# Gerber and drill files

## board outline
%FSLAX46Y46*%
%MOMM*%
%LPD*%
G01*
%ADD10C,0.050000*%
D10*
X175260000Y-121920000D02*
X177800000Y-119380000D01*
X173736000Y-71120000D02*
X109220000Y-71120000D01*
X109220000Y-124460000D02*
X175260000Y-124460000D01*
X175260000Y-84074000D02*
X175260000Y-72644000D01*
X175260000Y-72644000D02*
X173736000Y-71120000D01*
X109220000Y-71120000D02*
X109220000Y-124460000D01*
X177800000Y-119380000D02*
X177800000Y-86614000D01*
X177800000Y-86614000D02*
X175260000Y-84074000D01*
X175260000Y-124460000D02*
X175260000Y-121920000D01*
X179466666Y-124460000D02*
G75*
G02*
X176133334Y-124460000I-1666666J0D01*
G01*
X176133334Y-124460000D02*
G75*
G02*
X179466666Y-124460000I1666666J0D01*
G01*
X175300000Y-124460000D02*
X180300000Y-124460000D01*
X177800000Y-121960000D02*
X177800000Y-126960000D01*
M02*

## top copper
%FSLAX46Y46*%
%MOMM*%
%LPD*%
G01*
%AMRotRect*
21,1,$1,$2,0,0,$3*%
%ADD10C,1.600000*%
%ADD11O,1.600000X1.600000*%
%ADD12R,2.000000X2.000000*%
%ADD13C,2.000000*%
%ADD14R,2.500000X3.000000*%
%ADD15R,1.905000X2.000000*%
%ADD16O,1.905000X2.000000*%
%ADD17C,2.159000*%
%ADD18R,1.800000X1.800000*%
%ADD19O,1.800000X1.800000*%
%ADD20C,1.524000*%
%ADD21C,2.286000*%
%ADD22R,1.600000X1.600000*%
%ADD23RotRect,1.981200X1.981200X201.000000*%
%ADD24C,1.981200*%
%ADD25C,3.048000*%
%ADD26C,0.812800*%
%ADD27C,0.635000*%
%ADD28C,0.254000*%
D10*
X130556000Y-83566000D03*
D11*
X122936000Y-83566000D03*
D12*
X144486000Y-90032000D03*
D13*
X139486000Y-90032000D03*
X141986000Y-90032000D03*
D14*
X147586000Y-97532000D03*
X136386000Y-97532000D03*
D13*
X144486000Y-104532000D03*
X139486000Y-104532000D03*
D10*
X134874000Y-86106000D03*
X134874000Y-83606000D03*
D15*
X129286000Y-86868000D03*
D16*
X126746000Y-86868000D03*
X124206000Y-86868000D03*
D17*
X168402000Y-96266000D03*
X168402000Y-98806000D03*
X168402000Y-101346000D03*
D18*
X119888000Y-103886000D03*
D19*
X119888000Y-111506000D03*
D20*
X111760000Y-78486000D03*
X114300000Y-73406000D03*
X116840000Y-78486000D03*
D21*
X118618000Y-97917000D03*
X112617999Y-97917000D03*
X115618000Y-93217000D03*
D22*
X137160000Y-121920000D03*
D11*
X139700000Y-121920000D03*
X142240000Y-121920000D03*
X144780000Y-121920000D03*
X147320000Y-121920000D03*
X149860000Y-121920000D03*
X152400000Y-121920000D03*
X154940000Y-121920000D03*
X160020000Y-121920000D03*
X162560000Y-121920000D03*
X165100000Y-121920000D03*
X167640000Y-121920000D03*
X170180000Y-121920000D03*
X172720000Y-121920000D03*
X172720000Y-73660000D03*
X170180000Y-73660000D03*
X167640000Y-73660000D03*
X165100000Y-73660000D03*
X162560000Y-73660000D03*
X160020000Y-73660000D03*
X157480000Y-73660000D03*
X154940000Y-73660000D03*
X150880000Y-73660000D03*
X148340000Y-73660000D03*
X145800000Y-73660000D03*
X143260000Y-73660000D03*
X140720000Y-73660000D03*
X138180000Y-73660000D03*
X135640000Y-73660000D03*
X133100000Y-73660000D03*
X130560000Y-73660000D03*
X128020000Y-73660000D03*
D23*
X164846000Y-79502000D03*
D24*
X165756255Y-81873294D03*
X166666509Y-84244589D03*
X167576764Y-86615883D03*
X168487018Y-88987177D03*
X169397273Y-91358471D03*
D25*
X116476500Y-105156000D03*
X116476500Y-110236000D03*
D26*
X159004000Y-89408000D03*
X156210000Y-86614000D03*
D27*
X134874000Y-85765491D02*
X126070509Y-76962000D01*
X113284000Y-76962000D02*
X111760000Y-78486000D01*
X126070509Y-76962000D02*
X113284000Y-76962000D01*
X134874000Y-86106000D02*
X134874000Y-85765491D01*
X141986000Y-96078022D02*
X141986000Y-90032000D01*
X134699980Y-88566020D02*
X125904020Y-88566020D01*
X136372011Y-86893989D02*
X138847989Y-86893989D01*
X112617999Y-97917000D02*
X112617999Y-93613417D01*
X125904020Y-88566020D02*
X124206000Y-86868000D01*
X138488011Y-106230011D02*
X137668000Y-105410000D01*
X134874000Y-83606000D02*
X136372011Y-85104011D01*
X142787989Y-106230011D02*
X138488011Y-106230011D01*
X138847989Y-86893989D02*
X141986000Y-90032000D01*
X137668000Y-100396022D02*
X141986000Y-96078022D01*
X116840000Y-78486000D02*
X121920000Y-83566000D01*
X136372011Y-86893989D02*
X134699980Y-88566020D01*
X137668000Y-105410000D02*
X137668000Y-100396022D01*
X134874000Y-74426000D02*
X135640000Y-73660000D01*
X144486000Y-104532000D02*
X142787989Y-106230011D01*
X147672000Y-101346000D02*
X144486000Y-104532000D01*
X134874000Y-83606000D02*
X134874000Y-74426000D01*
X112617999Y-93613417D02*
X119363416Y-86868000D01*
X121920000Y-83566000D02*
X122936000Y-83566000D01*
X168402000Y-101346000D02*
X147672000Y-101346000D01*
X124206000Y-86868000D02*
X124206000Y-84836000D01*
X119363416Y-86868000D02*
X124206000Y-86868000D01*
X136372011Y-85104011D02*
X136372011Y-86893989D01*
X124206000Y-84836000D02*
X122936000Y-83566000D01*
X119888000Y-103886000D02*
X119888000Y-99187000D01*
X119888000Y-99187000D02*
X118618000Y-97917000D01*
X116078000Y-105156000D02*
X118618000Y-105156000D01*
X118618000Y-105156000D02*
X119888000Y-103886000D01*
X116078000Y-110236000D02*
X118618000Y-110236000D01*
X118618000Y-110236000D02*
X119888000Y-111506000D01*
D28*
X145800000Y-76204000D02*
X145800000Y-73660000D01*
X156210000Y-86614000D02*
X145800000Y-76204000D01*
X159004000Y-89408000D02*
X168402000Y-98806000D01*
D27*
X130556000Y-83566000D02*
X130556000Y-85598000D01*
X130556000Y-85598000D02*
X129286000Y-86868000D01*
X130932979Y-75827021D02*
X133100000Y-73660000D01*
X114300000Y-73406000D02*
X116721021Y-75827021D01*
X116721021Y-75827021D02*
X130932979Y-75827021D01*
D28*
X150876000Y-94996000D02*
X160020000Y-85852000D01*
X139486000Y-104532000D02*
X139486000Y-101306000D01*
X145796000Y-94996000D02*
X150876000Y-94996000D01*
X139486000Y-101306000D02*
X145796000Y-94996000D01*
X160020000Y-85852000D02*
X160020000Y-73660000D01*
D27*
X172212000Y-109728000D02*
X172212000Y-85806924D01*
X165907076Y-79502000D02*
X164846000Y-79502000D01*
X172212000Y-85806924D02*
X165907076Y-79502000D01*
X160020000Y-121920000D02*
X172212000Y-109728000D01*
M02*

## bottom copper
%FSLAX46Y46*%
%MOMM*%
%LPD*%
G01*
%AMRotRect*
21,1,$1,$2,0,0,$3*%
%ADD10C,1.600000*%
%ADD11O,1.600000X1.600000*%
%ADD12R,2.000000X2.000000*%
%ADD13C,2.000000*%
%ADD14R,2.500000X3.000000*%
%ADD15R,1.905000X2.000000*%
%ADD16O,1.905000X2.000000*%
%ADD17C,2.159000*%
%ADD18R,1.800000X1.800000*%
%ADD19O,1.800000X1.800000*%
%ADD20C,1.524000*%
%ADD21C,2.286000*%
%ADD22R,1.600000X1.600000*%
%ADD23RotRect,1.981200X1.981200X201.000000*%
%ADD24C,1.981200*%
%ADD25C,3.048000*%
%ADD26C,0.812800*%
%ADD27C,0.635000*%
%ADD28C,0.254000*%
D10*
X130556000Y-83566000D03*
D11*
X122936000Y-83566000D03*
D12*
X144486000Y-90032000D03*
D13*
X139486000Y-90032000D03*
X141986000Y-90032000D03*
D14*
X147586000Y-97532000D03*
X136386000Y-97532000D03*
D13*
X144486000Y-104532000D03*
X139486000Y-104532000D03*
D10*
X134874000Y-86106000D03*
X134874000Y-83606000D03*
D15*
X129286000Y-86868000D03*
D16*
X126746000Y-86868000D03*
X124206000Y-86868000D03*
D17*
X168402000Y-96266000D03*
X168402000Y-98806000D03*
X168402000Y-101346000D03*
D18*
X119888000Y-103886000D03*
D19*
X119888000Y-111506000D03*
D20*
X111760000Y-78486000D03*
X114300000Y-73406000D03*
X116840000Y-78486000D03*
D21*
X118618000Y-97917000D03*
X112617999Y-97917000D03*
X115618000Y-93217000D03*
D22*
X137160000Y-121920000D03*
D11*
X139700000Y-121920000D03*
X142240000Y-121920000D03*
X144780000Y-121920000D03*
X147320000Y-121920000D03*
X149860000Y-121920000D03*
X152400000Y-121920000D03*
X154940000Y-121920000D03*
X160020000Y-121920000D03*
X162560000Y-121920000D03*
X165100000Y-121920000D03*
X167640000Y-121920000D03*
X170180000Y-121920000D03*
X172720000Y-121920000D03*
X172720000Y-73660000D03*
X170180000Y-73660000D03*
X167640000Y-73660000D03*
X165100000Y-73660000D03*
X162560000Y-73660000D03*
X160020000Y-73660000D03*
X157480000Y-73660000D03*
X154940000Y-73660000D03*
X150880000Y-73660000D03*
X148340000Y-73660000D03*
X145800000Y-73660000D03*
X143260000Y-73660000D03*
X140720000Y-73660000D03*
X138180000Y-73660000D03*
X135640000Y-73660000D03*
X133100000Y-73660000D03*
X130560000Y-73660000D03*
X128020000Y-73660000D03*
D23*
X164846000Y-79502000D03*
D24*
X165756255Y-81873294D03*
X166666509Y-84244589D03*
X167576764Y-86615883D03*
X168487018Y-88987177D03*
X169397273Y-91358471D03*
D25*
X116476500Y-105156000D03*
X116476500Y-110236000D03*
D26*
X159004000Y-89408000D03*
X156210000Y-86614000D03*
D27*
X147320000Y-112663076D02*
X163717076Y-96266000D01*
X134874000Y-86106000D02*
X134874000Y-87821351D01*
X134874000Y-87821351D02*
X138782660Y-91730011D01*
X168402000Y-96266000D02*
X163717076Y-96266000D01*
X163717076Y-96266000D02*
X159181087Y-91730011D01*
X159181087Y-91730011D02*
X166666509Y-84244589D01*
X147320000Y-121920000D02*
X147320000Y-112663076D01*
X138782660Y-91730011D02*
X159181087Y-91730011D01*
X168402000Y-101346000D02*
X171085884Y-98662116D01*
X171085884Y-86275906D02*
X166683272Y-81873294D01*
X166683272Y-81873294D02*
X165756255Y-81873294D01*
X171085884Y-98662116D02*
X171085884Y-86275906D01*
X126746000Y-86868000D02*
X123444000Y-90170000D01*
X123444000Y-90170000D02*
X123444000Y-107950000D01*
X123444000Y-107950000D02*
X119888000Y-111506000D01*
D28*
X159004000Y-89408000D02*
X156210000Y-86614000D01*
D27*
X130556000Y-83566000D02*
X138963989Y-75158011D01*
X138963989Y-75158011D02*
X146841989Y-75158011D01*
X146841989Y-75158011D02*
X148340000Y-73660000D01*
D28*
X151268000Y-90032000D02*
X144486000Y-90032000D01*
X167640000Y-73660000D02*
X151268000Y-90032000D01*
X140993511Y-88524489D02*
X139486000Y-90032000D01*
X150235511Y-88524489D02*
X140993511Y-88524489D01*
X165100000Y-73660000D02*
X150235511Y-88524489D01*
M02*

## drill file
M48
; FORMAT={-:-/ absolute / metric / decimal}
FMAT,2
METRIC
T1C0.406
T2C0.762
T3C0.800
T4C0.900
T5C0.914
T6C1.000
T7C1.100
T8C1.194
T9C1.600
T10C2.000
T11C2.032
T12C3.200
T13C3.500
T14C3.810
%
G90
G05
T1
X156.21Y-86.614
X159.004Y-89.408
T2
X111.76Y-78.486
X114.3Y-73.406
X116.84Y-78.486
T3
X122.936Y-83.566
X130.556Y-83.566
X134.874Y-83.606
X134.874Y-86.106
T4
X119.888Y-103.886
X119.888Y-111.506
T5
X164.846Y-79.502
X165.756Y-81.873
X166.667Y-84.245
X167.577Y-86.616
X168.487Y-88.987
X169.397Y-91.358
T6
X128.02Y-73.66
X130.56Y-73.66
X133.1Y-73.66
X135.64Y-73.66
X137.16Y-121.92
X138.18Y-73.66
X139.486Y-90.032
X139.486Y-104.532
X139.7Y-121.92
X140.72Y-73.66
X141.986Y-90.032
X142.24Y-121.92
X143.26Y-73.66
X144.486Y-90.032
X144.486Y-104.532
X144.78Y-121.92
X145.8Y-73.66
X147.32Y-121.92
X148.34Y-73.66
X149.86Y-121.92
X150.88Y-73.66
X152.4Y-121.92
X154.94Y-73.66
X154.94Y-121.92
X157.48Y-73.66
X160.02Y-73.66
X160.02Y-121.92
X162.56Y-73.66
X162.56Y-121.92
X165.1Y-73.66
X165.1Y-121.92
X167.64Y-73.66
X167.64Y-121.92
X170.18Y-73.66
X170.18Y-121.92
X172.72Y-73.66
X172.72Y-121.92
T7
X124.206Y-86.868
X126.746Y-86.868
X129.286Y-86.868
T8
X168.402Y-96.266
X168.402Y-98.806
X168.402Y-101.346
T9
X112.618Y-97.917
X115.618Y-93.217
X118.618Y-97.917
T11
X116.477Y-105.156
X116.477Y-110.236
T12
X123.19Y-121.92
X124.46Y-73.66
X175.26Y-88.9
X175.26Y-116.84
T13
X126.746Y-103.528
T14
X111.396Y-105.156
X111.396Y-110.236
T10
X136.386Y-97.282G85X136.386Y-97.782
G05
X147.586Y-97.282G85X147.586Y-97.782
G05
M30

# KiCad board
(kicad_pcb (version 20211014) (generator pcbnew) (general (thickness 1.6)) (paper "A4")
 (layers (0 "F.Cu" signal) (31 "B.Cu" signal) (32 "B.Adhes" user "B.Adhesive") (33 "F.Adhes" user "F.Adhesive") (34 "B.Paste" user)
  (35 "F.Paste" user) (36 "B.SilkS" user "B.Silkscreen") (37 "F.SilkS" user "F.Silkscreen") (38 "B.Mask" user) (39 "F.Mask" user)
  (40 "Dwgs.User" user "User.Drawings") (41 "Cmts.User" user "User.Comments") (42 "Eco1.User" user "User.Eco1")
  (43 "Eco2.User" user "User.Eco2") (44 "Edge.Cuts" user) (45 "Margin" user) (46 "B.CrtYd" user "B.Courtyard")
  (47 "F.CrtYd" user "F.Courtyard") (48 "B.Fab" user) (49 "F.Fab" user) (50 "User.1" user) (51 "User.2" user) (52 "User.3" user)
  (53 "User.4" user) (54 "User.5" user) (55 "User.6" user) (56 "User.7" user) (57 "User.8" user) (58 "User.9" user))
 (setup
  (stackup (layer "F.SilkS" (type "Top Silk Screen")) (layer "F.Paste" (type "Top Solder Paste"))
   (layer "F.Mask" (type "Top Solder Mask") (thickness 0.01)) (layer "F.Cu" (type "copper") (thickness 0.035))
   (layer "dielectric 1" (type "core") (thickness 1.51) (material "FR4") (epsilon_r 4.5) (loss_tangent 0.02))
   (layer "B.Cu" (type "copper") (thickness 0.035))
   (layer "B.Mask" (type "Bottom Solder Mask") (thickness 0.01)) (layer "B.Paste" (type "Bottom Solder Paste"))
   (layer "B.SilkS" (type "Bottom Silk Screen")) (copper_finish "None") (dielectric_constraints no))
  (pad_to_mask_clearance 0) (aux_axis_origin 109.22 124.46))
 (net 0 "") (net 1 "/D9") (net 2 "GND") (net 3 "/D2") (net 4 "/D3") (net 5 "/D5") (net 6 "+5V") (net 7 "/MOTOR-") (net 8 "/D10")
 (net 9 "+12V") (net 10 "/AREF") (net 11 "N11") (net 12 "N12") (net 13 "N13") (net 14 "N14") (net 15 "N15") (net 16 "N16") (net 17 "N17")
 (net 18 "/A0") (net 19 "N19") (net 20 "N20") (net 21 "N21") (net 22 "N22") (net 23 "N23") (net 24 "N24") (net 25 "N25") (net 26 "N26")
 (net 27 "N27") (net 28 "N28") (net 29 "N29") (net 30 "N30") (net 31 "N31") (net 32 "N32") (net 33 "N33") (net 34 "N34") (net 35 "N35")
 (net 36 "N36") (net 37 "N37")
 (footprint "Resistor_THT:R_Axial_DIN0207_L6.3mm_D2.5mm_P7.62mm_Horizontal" (layer "F.Cu") (at 130.556 83.566 180)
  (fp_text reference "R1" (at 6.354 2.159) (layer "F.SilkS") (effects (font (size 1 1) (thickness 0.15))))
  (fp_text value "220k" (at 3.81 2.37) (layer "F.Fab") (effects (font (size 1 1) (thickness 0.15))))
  (pad "1" thru_hole circle (at 0 0 180) (size 1.6 1.6) (drill 0.8) (layers *.Cu *.Mask) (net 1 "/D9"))
  (pad "2" thru_hole oval (at 7.62 0 180) (size 1.6 1.6) (drill 0.8) (layers *.Cu *.Mask) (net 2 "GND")))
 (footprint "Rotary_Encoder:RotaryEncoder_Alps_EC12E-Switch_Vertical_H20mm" (layer "F.Cu") (at 144.486 90.032 -90)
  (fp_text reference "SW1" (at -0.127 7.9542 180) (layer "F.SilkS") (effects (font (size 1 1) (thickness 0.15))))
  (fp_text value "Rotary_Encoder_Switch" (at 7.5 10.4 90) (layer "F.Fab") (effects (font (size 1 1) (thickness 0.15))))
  (pad "A" thru_hole rect (at 0 0 270) (size 2 2) (drill 1) (layers *.Cu *.Mask) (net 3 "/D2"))
  (pad "B" thru_hole circle (at 0 5 270) (size 2 2) (drill 1) (layers *.Cu *.Mask) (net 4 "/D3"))
  (pad "C" thru_hole circle (at 0 2.5 270) (size 2 2) (drill 1) (layers *.Cu *.Mask) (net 2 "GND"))
  (pad "MP" thru_hole rect (at 7.5 -3.1 270) (size 3 2.5) (drill oval 2.5 2) (layers *.Cu *.Mask))
  (pad "MP" thru_hole rect (at 7.5 8.1 270) (size 3 2.5) (drill oval 2.5 2) (layers *.Cu *.Mask))
  (pad "S1" thru_hole circle (at 14.5 0 270) (size 2 2) (drill 1) (layers *.Cu *.Mask) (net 2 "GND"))
  (pad "S2" thru_hole circle (at 14.5 5 270) (size 2 2) (drill 1) (layers *.Cu *.Mask) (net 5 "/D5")))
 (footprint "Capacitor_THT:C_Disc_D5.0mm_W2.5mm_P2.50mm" (layer "F.Cu") (at 134.874 86.106 90)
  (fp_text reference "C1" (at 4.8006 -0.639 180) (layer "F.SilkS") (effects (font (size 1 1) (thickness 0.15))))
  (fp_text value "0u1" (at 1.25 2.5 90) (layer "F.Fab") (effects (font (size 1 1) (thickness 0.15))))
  (pad "1" thru_hole circle (at 0 0 90) (size 1.6 1.6) (drill 0.8) (layers *.Cu *.Mask) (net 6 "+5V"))
  (pad "2" thru_hole circle (at 2.5 0 90) (size 1.6 1.6) (drill 0.8) (layers *.Cu *.Mask) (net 2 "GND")))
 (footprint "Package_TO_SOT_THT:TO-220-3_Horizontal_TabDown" (layer "F.Cu") (at 129.286 86.868 180)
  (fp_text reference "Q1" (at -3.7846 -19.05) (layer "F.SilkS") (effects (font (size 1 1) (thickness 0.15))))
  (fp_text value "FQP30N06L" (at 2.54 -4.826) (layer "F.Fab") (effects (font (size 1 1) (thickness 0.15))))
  (pad "" np_thru_hole oval (at 2.54 -16.66 180) (size 3.5 3.5) (drill 3.5) (layers *.Cu *.Mask))
  (pad "1" thru_hole rect (at 0 0 180) (size 1.905 2) (drill 1.1) (layers *.Cu *.Mask) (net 1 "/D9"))
  (pad "2" thru_hole oval (at 2.54 0 180) (size 1.905 2) (drill 1.1) (layers *.Cu *.Mask) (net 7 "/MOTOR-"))
  (pad "3" thru_hole oval (at 5.08 0 180) (size 1.905 2) (drill 1.1) (layers *.Cu *.Mask) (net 2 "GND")))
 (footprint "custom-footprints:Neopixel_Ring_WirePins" (layer "F.Cu") (at 168.402 96.266)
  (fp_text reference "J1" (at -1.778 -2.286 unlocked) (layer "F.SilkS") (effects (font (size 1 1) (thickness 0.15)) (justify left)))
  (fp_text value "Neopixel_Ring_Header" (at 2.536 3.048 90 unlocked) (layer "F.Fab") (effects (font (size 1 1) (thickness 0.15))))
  (pad "1" thru_hole circle (at 0 0) (size 2.159 2.159) (drill 1.1938) (layers *.Cu *.Mask) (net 6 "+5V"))
  (pad "2" thru_hole circle (at 0 2.54) (size 2.159 2.159) (drill 1.1938) (layers *.Cu *.Mask) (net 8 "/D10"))
  (pad "3" thru_hole circle (at 0 5.08) (size 2.159 2.159) (drill 1.1938) (layers *.Cu *.Mask) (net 2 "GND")))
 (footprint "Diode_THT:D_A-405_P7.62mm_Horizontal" (layer "F.Cu") (at 119.888 103.886 -90)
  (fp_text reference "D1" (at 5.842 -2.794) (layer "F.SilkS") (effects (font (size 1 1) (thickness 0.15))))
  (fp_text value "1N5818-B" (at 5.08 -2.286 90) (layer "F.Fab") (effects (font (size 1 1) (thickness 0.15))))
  (pad "1" thru_hole rect (at 0 0 270) (size 1.8 1.8) (drill 0.9) (layers *.Cu *.Mask) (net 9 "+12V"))
  (pad "2" thru_hole oval (at 7.62 0 270) (size 1.8 1.8) (drill 0.9) (layers *.Cu *.Mask) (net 7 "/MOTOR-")))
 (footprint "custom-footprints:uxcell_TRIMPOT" (layer "F.Cu") (at 111.76 78.486)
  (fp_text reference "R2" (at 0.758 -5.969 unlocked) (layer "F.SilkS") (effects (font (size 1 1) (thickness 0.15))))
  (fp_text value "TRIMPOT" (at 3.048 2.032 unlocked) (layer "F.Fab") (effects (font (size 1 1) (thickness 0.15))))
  (pad "1" thru_hole circle (at 0 0) (size 1.524 1.524) (drill 0.762) (layers *.Cu *.Mask) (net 6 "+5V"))
  (pad "2" thru_hole circle (at 2.54 -5.08) (size 1.524 1.524) (drill 0.762) (layers *.Cu *.Mask) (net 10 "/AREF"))
  (pad "3" thru_hole circle (at 5.08 0) (size 1.524 1.524) (drill 0.762) (layers *.Cu *.Mask) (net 2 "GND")))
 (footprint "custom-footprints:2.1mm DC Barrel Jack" (layer "B.Cu") (at 118.618 97.917 -90)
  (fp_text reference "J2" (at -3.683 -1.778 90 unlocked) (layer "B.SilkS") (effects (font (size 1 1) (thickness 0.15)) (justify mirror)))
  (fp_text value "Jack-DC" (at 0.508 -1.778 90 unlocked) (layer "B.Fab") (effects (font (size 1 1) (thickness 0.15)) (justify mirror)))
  (pad "1" thru_hole circle (at 0 0 270) (size 2.286 2.286) (drill 1.6002) (layers *.Cu *.Mask) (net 9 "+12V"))
  (pad "2" thru_hole circle (at 0 6.000001 270) (size 2.286 2.286) (drill 1.6002) (layers *.Cu *.Mask) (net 2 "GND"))
  (pad "3" thru_hole circle (at -4.7 3 270) (size 2.286 2.286) (drill 1.6002) (layers *.Cu *.Mask)))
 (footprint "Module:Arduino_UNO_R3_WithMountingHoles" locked (layer "B.Cu") (at 137.16 121.92)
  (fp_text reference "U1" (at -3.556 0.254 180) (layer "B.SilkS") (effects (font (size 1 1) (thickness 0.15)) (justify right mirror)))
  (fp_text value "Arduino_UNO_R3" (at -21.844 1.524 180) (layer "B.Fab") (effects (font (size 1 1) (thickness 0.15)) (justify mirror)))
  (pad "" np_thru_hole circle locked (at -12.7 -48.26 270) (size 3.2 3.2) (drill 3.2) (layers *.Cu *.Mask))
  (pad "" np_thru_hole circle locked (at 38.1 -5.08 270) (size 3.2 3.2) (drill 3.2) (layers *.Cu *.Mask))
  (pad "" np_thru_hole circle locked (at -13.97 0 270) (size 3.2 3.2) (drill 3.2) (layers *.Cu *.Mask))
  (pad "" np_thru_hole circle locked (at 38.1 -33.02 270) (size 3.2 3.2) (drill 3.2) (layers *.Cu *.Mask))
  (pad "1" thru_hole rect locked (at 0 0 270) (size 1.6 1.6) (drill 1) (layers *.Cu *.Mask) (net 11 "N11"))
  (pad "2" thru_hole oval locked (at 2.54 0 270) (size 1.6 1.6) (drill 1) (layers *.Cu *.Mask) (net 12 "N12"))
  (pad "3" thru_hole oval locked (at 5.08 0 270) (size 1.6 1.6) (drill 1) (layers *.Cu *.Mask) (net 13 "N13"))
  (pad "4" thru_hole oval locked (at 7.62 0 270) (size 1.6 1.6) (drill 1) (layers *.Cu *.Mask) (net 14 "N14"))
  (pad "5" thru_hole oval locked (at 10.16 0 270) (size 1.6 1.6) (drill 1) (layers *.Cu *.Mask) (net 6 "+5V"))
  (pad "6" thru_hole oval locked (at 12.7 0 270) (size 1.6 1.6) (drill 1) (layers *.Cu *.Mask) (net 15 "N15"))
  (pad "7" thru_hole oval locked (at 15.24 0 270) (size 1.6 1.6) (drill 1) (layers *.Cu *.Mask) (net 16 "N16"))
  (pad "8" thru_hole oval locked (at 17.78 0 270) (size 1.6 1.6) (drill 1) (layers *.Cu *.Mask) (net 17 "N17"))
  (pad "9" thru_hole oval locked (at 22.86 0 270) (size 1.6 1.6) (drill 1) (layers *.Cu *.Mask) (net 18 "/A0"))
  (pad "10" thru_hole oval locked (at 25.4 0 270) (size 1.6 1.6) (drill 1) (layers *.Cu *.Mask) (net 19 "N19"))
  (pad "11" thru_hole oval locked (at 27.94 0 270) (size 1.6 1.6) (drill 1) (layers *.Cu *.Mask) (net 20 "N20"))
  (pad "12" thru_hole oval locked (at 30.48 0 270) (size 1.6 1.6) (drill 1) (layers *.Cu *.Mask) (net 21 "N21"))
  (pad "13" thru_hole oval locked (at 33.02 0 270) (size 1.6 1.6) (drill 1) (layers *.Cu *.Mask) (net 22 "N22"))
  (pad "14" thru_hole oval locked (at 35.56 0 270) (size 1.6 1.6) (drill 1) (layers *.Cu *.Mask) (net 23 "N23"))
  (pad "15" thru_hole oval locked (at 35.56 -48.26 270) (size 1.6 1.6) (drill 1) (layers *.Cu *.Mask) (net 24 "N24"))
  (pad "16" thru_hole oval locked (at 33.02 -48.26 270) (size 1.6 1.6) (drill 1) (layers *.Cu *.Mask) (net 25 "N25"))
  (pad "17" thru_hole oval locked (at 30.48 -48.26 270) (size 1.6 1.6) (drill 1) (layers *.Cu *.Mask) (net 3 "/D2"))
  (pad "18" thru_hole oval locked (at 27.94 -48.26 270) (size 1.6 1.6) (drill 1) (layers *.Cu *.Mask) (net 4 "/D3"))
  (pad "19" thru_hole oval locked (at 25.4 -48.26 270) (size 1.6 1.6) (drill 1) (layers *.Cu *.Mask) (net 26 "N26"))
  (pad "20" thru_hole oval locked (at 22.86 -48.26 270) (size 1.6 1.6) (drill 1) (layers *.Cu *.Mask) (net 5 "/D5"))
  (pad "21" thru_hole oval locked (at 20.32 -48.26 270) (size 1.6 1.6) (drill 1) (layers *.Cu *.Mask) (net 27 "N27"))
  (pad "22" thru_hole oval locked (at 17.78 -48.26 270) (size 1.6 1.6) (drill 1) (layers *.Cu *.Mask) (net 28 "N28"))
  (pad "23" thru_hole oval locked (at 13.72 -48.26 270) (size 1.6 1.6) (drill 1) (layers *.Cu *.Mask) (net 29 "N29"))
  (pad "24" thru_hole oval locked (at 11.18 -48.26 270) (size 1.6 1.6) (drill 1) (layers *.Cu *.Mask) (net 1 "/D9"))
  (pad "25" thru_hole oval locked (at 8.64 -48.26 270) (size 1.6 1.6) (drill 1) (layers *.Cu *.Mask) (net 8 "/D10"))
  (pad "26" thru_hole oval locked (at 6.1 -48.26 270) (size 1.6 1.6) (drill 1) (layers *.Cu *.Mask) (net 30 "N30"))
  (pad "27" thru_hole oval locked (at 3.56 -48.26 270) (size 1.6 1.6) (drill 1) (layers *.Cu *.Mask) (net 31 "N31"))
  (pad "28" thru_hole oval locked (at 1.02 -48.26 270) (size 1.6 1.6) (drill 1) (layers *.Cu *.Mask) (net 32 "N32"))
  (pad "29" thru_hole oval locked (at -1.52 -48.26 270) (size 1.6 1.6) (drill 1) (layers *.Cu *.Mask) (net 2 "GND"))
  (pad "30" thru_hole oval locked (at -4.06 -48.26 270) (size 1.6 1.6) (drill 1) (layers *.Cu *.Mask) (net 10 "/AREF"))
  (pad "31" thru_hole oval locked (at -6.6 -48.26 270) (size 1.6 1.6) (drill 1) (layers *.Cu *.Mask) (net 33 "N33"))
  (pad "32" thru_hole oval locked (at -9.14 -48.26 270) (size 1.6 1.6) (drill 1) (layers *.Cu *.Mask) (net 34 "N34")))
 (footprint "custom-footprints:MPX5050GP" (layer "B.Cu") (at 164.846 79.502 -159)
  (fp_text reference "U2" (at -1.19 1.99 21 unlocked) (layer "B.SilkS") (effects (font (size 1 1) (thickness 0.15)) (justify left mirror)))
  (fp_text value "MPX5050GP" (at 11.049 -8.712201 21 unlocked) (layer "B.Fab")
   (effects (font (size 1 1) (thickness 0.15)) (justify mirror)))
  (pad "1" thru_hole rect (at 0 0 201) (size 1.9812 1.9812) (drill 0.9144) (layers *.Cu *.Mask) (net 18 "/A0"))
  (pad "2" thru_hole circle (at 0 -2.54 201) (size 1.9812 1.9812) (drill 0.9144) (layers *.Cu *.Mask) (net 2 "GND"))
  (pad "3" thru_hole circle (at 0 -5.08 201) (size 1.9812 1.9812) (drill 0.9144) (layers *.Cu *.Mask) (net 6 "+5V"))
  (pad "4" thru_hole circle (at 0 -7.62 201) (size 1.9812 1.9812) (drill 0.9144) (layers *.Cu *.Mask) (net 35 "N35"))
  (pad "5" thru_hole circle (at 0 -10.16 201) (size 1.9812 1.9812) (drill 0.9144) (layers *.Cu *.Mask) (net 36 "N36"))
  (pad "6" thru_hole circle (at 0 -12.7 201) (size 1.9812 1.9812) (drill 0.9144) (layers *.Cu *.Mask) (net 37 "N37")))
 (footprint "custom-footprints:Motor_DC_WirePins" (layer "B.Cu") (at 116.4765 105.156 180)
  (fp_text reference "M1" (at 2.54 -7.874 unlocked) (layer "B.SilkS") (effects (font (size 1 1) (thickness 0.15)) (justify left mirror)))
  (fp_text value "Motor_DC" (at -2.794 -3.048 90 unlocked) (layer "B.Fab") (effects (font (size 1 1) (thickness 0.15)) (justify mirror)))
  (pad "" np_thru_hole circle (at 5.08 0 180) (size 3.302 3.302) (drill 3.81) (layers *.Mask))
  (pad "" np_thru_hole circle (at 5.08 -5.08 180) (size 3.302 3.302) (drill 3.81) (layers *.Mask))
  (pad "1" thru_hole circle (at 0 0 180) (size 3.048 3.048) (drill 2.032) (layers *.Cu *.Mask) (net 9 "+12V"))
  (pad "2" thru_hole circle (at 0 -5.08 180) (size 3.048 3.048) (drill 2.032) (layers *.Cu *.Mask) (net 7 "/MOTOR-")))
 (gr_line (start 175.26 121.92) (end 177.8 119.38) (layer "Edge.Cuts") (width 0.05))
 (gr_line (start 173.736 71.12) (end 109.22 71.12) (layer "Edge.Cuts") (width 0.05))
 (gr_line (start 109.22 124.46) (end 175.26 124.46) (layer "Edge.Cuts") (width 0.05))
 (gr_line (start 175.26 84.074) (end 175.26 72.644) (layer "Edge.Cuts") (width 0.05))
 (gr_line (start 175.26 72.644) (end 173.736 71.12) (layer "Edge.Cuts") (width 0.05))
 (gr_line (start 109.22 71.12) (end 109.22 124.46) (layer "Edge.Cuts") (width 0.05))
 (gr_line (start 177.8 119.38) (end 177.8 86.614) (layer "Edge.Cuts") (width 0.05))
 (gr_line (start 177.8 86.614) (end 175.26 84.074) (layer "Edge.Cuts") (width 0.05))
 (gr_line (start 175.26 124.46) (end 175.26 121.92) (layer "Edge.Cuts") (width 0.05))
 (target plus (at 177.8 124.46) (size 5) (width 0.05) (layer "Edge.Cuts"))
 (segment (start 134.874 85.765491) (end 126.070509 76.962) (width 0.635) (layer "F.Cu") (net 6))
 (segment (start 113.284 76.962) (end 111.76 78.486) (width 0.635) (layer "F.Cu") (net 6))
 (segment (start 126.070509 76.962) (end 113.284 76.962) (width 0.635) (layer "F.Cu") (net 6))
 (segment (start 134.874 86.106) (end 134.874 85.765491) (width 0.635) (layer "F.Cu") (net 6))
 (segment (start 147.32 112.663076) (end 163.717076 96.266) (width 0.635) (layer "B.Cu") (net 6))
 (segment (start 134.874 86.106) (end 134.874 87.821351) (width 0.635) (layer "B.Cu") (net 6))
 (segment (start 134.874 87.821351) (end 138.78266 91.730011) (width 0.635) (layer "B.Cu") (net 6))
 (segment (start 168.402 96.266) (end 163.717076 96.266) (width 0.635) (layer "B.Cu") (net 6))
 (segment (start 163.717076 96.266) (end 159.181087 91.730011) (width 0.635) (layer "B.Cu") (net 6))
 (segment (start 159.181087 91.730011) (end 166.666509 84.244589) (width 0.635) (layer "B.Cu") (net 6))
 (segment (start 147.32 121.92) (end 147.32 112.663076) (width 0.635) (layer "B.Cu") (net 6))
 (segment (start 138.78266 91.730011) (end 159.181087 91.730011) (width 0.635) (layer "B.Cu") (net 6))
 (segment (start 141.986 96.078022) (end 141.986 90.032) (width 0.635) (layer "F.Cu") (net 2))
 (segment (start 134.69998 88.56602) (end 125.90402 88.56602) (width 0.635) (layer "F.Cu") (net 2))
 (segment (start 136.372011 86.893989) (end 138.847989 86.893989) (width 0.635) (layer "F.Cu") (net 2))
 (segment (start 112.617999 97.917) (end 112.617999 93.613417) (width 0.635) (layer "F.Cu") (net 2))
 (segment (start 125.90402 88.56602) (end 124.206 86.868) (width 0.635) (layer "F.Cu") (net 2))
 (segment (start 138.488011 106.230011) (end 137.668 105.41) (width 0.635) (layer "F.Cu") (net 2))
 (segment (start 134.874 83.606) (end 136.372011 85.104011) (width 0.635) (layer "F.Cu") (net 2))
 (segment (start 142.787989 106.230011) (end 138.488011 106.230011) (width 0.635) (layer "F.Cu") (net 2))
 (segment (start 138.847989 86.893989) (end 141.986 90.032) (width 0.635) (layer "F.Cu") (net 2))
 (segment (start 137.668 100.396022) (end 141.986 96.078022) (width 0.635) (layer "F.Cu") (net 2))
 (segment (start 116.84 78.486) (end 121.92 83.566) (width 0.635) (layer "F.Cu") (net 2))
 (segment (start 136.372011 86.893989) (end 134.69998 88.56602) (width 0.635) (layer "F.Cu") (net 2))
 (segment (start 137.668 105.41) (end 137.668 100.396022) (width 0.635) (layer "F.Cu") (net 2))
 (segment (start 134.874 74.426) (end 135.64 73.66) (width 0.635) (layer "F.Cu") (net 2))
 (segment (start 144.486 104.532) (end 142.787989 106.230011) (width 0.635) (layer "F.Cu") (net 2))
 (segment (start 147.672 101.346) (end 144.486 104.532) (width 0.635) (layer "F.Cu") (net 2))
 (segment (start 134.874 83.606) (end 134.874 74.426) (width 0.635) (layer "F.Cu") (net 2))
 (segment (start 112.617999 93.613417) (end 119.363416 86.868) (width 0.635) (layer "F.Cu") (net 2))
 (segment (start 121.92 83.566) (end 122.936 83.566) (width 0.635) (layer "F.Cu") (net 2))
 (segment (start 168.402 101.346) (end 147.672 101.346) (width 0.635) (layer "F.Cu") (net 2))
 (segment (start 124.206 86.868) (end 124.206 84.836) (width 0.635) (layer "F.Cu") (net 2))
 (segment (start 119.363416 86.868) (end 124.206 86.868) (width 0.635) (layer "F.Cu") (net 2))
 (segment (start 136.372011 85.104011) (end 136.372011 86.893989) (width 0.635) (layer "F.Cu") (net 2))
 (segment (start 124.206 84.836) (end 122.936 83.566) (width 0.635) (layer "F.Cu") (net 2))
 (segment (start 168.402 101.346) (end 171.085884 98.662116) (width 0.635) (layer "B.Cu") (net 2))
 (segment (start 171.085884 86.275906) (end 166.683272 81.873294) (width 0.635) (layer "B.Cu") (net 2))
 (segment (start 166.683272 81.873294) (end 165.756255 81.873294) (width 0.635) (layer "B.Cu") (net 2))
 (segment (start 171.085884 98.662116) (end 171.085884 86.275906) (width 0.635) (layer "B.Cu") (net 2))
 (segment (start 119.888 103.886) (end 119.888 99.187) (width 0.635) (layer "F.Cu") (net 9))
 (segment (start 119.888 99.187) (end 118.618 97.917) (width 0.635) (layer "F.Cu") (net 9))
 (segment (start 116.078 105.156) (end 118.618 105.156) (width 0.635) (layer "F.Cu") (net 9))
 (segment (start 118.618 105.156) (end 119.888 103.886) (width 0.635) (layer "F.Cu") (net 9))
 (segment (start 116.078 110.236) (end 118.618 110.236) (width 0.635) (layer "F.Cu") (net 7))
 (segment (start 118.618 110.236) (end 119.888 111.506) (width 0.635) (layer "F.Cu") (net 7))
 (segment (start 126.746 86.868) (end 123.444 90.17) (width 0.635) (layer "B.Cu") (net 7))
 (segment (start 123.444 90.17) (end 123.444 107.95) (width 0.635) (layer "B.Cu") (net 7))
 (segment (start 123.444 107.95) (end 119.888 111.506) (width 0.635) (layer "B.Cu") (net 7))
 (segment (start 145.8 76.204) (end 145.8 73.66) (width 0.254) (layer "F.Cu") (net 8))
 (segment (start 156.21 86.614) (end 145.8 76.204) (width 0.254) (layer "F.Cu") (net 8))
 (segment (start 159.004 89.408) (end 168.402 98.806) (width 0.254) (layer "F.Cu") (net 8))
 (via (at 159.004 89.408) (size 0.8128) (drill 0.4064) (layers "F.Cu" "B.Cu") (free) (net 8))
 (via (at 156.21 86.614) (size 0.8128) (drill 0.4064) (layers "F.Cu" "B.Cu") (free) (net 8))
 (segment (start 159.004 89.408) (end 156.21 86.614) (width 0.254) (layer "B.Cu") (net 8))
 (segment (start 130.556 83.566) (end 130.556 85.598) (width 0.635) (layer "F.Cu") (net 1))
 (segment (start 130.556 85.598) (end 129.286 86.868) (width 0.635) (layer "F.Cu") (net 1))
 (segment (start 130.556 83.566) (end 138.963989 75.158011) (width 0.635) (layer "B.Cu") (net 1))
 (segment (start 138.963989 75.158011) (end 146.841989 75.158011) (width 0.635) (layer "B.Cu") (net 1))
 (segment (start 146.841989 75.158011) (end 148.34 73.66) (width 0.635) (layer "B.Cu") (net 1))
 (segment (start 130.932979 75.827021) (end 133.1 73.66) (width 0.635) (layer "F.Cu") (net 10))
 (segment (start 114.3 73.406) (end 116.721021 75.827021) (width 0.635) (layer "F.Cu") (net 10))
 (segment (start 116.721021 75.827021) (end 130.932979 75.827021) (width 0.635) (layer "F.Cu") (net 10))
 (segment (start 151.268 90.032) (end 144.486 90.032) (width 0.254) (layer "B.Cu") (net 3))
 (segment (start 167.64 73.66) (end 151.268 90.032) (width 0.254) (layer "B.Cu") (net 3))
 (segment (start 140.993511 88.524489) (end 139.486 90.032) (width 0.254) (layer "B.Cu") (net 4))
 (segment (start 150.235511 88.524489) (end 140.993511 88.524489) (width 0.254) (layer "B.Cu") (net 4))
 (segment (start 165.1 73.66) (end 150.235511 88.524489) (width 0.254) (layer "B.Cu") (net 4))
 (segment (start 150.876 94.996) (end 160.02 85.852) (width 0.254) (layer "F.Cu") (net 5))
 (segment (start 139.486 104.532) (end 139.486 101.306) (width 0.254) (layer "F.Cu") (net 5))
 (segment (start 145.796 94.996) (end 150.876 94.996) (width 0.254) (layer "F.Cu") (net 5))
 (segment (start 139.486 101.306) (end 145.796 94.996) (width 0.254) (layer "F.Cu") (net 5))
 (segment (start 160.02 85.852) (end 160.02 73.66) (width 0.254) (layer "F.Cu") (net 5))
 (segment (start 172.212 109.728) (end 172.212 85.806924) (width 0.635) (layer "F.Cu") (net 18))
 (segment (start 165.907076 79.502) (end 164.846 79.502) (width 0.635) (layer "F.Cu") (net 18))
 (segment (start 172.212 85.806924) (end 165.907076 79.502) (width 0.635) (layer "F.Cu") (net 18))
 (segment (start 160.02 121.92) (end 172.212 109.728) (width 0.635) (layer "F.Cu") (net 18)))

